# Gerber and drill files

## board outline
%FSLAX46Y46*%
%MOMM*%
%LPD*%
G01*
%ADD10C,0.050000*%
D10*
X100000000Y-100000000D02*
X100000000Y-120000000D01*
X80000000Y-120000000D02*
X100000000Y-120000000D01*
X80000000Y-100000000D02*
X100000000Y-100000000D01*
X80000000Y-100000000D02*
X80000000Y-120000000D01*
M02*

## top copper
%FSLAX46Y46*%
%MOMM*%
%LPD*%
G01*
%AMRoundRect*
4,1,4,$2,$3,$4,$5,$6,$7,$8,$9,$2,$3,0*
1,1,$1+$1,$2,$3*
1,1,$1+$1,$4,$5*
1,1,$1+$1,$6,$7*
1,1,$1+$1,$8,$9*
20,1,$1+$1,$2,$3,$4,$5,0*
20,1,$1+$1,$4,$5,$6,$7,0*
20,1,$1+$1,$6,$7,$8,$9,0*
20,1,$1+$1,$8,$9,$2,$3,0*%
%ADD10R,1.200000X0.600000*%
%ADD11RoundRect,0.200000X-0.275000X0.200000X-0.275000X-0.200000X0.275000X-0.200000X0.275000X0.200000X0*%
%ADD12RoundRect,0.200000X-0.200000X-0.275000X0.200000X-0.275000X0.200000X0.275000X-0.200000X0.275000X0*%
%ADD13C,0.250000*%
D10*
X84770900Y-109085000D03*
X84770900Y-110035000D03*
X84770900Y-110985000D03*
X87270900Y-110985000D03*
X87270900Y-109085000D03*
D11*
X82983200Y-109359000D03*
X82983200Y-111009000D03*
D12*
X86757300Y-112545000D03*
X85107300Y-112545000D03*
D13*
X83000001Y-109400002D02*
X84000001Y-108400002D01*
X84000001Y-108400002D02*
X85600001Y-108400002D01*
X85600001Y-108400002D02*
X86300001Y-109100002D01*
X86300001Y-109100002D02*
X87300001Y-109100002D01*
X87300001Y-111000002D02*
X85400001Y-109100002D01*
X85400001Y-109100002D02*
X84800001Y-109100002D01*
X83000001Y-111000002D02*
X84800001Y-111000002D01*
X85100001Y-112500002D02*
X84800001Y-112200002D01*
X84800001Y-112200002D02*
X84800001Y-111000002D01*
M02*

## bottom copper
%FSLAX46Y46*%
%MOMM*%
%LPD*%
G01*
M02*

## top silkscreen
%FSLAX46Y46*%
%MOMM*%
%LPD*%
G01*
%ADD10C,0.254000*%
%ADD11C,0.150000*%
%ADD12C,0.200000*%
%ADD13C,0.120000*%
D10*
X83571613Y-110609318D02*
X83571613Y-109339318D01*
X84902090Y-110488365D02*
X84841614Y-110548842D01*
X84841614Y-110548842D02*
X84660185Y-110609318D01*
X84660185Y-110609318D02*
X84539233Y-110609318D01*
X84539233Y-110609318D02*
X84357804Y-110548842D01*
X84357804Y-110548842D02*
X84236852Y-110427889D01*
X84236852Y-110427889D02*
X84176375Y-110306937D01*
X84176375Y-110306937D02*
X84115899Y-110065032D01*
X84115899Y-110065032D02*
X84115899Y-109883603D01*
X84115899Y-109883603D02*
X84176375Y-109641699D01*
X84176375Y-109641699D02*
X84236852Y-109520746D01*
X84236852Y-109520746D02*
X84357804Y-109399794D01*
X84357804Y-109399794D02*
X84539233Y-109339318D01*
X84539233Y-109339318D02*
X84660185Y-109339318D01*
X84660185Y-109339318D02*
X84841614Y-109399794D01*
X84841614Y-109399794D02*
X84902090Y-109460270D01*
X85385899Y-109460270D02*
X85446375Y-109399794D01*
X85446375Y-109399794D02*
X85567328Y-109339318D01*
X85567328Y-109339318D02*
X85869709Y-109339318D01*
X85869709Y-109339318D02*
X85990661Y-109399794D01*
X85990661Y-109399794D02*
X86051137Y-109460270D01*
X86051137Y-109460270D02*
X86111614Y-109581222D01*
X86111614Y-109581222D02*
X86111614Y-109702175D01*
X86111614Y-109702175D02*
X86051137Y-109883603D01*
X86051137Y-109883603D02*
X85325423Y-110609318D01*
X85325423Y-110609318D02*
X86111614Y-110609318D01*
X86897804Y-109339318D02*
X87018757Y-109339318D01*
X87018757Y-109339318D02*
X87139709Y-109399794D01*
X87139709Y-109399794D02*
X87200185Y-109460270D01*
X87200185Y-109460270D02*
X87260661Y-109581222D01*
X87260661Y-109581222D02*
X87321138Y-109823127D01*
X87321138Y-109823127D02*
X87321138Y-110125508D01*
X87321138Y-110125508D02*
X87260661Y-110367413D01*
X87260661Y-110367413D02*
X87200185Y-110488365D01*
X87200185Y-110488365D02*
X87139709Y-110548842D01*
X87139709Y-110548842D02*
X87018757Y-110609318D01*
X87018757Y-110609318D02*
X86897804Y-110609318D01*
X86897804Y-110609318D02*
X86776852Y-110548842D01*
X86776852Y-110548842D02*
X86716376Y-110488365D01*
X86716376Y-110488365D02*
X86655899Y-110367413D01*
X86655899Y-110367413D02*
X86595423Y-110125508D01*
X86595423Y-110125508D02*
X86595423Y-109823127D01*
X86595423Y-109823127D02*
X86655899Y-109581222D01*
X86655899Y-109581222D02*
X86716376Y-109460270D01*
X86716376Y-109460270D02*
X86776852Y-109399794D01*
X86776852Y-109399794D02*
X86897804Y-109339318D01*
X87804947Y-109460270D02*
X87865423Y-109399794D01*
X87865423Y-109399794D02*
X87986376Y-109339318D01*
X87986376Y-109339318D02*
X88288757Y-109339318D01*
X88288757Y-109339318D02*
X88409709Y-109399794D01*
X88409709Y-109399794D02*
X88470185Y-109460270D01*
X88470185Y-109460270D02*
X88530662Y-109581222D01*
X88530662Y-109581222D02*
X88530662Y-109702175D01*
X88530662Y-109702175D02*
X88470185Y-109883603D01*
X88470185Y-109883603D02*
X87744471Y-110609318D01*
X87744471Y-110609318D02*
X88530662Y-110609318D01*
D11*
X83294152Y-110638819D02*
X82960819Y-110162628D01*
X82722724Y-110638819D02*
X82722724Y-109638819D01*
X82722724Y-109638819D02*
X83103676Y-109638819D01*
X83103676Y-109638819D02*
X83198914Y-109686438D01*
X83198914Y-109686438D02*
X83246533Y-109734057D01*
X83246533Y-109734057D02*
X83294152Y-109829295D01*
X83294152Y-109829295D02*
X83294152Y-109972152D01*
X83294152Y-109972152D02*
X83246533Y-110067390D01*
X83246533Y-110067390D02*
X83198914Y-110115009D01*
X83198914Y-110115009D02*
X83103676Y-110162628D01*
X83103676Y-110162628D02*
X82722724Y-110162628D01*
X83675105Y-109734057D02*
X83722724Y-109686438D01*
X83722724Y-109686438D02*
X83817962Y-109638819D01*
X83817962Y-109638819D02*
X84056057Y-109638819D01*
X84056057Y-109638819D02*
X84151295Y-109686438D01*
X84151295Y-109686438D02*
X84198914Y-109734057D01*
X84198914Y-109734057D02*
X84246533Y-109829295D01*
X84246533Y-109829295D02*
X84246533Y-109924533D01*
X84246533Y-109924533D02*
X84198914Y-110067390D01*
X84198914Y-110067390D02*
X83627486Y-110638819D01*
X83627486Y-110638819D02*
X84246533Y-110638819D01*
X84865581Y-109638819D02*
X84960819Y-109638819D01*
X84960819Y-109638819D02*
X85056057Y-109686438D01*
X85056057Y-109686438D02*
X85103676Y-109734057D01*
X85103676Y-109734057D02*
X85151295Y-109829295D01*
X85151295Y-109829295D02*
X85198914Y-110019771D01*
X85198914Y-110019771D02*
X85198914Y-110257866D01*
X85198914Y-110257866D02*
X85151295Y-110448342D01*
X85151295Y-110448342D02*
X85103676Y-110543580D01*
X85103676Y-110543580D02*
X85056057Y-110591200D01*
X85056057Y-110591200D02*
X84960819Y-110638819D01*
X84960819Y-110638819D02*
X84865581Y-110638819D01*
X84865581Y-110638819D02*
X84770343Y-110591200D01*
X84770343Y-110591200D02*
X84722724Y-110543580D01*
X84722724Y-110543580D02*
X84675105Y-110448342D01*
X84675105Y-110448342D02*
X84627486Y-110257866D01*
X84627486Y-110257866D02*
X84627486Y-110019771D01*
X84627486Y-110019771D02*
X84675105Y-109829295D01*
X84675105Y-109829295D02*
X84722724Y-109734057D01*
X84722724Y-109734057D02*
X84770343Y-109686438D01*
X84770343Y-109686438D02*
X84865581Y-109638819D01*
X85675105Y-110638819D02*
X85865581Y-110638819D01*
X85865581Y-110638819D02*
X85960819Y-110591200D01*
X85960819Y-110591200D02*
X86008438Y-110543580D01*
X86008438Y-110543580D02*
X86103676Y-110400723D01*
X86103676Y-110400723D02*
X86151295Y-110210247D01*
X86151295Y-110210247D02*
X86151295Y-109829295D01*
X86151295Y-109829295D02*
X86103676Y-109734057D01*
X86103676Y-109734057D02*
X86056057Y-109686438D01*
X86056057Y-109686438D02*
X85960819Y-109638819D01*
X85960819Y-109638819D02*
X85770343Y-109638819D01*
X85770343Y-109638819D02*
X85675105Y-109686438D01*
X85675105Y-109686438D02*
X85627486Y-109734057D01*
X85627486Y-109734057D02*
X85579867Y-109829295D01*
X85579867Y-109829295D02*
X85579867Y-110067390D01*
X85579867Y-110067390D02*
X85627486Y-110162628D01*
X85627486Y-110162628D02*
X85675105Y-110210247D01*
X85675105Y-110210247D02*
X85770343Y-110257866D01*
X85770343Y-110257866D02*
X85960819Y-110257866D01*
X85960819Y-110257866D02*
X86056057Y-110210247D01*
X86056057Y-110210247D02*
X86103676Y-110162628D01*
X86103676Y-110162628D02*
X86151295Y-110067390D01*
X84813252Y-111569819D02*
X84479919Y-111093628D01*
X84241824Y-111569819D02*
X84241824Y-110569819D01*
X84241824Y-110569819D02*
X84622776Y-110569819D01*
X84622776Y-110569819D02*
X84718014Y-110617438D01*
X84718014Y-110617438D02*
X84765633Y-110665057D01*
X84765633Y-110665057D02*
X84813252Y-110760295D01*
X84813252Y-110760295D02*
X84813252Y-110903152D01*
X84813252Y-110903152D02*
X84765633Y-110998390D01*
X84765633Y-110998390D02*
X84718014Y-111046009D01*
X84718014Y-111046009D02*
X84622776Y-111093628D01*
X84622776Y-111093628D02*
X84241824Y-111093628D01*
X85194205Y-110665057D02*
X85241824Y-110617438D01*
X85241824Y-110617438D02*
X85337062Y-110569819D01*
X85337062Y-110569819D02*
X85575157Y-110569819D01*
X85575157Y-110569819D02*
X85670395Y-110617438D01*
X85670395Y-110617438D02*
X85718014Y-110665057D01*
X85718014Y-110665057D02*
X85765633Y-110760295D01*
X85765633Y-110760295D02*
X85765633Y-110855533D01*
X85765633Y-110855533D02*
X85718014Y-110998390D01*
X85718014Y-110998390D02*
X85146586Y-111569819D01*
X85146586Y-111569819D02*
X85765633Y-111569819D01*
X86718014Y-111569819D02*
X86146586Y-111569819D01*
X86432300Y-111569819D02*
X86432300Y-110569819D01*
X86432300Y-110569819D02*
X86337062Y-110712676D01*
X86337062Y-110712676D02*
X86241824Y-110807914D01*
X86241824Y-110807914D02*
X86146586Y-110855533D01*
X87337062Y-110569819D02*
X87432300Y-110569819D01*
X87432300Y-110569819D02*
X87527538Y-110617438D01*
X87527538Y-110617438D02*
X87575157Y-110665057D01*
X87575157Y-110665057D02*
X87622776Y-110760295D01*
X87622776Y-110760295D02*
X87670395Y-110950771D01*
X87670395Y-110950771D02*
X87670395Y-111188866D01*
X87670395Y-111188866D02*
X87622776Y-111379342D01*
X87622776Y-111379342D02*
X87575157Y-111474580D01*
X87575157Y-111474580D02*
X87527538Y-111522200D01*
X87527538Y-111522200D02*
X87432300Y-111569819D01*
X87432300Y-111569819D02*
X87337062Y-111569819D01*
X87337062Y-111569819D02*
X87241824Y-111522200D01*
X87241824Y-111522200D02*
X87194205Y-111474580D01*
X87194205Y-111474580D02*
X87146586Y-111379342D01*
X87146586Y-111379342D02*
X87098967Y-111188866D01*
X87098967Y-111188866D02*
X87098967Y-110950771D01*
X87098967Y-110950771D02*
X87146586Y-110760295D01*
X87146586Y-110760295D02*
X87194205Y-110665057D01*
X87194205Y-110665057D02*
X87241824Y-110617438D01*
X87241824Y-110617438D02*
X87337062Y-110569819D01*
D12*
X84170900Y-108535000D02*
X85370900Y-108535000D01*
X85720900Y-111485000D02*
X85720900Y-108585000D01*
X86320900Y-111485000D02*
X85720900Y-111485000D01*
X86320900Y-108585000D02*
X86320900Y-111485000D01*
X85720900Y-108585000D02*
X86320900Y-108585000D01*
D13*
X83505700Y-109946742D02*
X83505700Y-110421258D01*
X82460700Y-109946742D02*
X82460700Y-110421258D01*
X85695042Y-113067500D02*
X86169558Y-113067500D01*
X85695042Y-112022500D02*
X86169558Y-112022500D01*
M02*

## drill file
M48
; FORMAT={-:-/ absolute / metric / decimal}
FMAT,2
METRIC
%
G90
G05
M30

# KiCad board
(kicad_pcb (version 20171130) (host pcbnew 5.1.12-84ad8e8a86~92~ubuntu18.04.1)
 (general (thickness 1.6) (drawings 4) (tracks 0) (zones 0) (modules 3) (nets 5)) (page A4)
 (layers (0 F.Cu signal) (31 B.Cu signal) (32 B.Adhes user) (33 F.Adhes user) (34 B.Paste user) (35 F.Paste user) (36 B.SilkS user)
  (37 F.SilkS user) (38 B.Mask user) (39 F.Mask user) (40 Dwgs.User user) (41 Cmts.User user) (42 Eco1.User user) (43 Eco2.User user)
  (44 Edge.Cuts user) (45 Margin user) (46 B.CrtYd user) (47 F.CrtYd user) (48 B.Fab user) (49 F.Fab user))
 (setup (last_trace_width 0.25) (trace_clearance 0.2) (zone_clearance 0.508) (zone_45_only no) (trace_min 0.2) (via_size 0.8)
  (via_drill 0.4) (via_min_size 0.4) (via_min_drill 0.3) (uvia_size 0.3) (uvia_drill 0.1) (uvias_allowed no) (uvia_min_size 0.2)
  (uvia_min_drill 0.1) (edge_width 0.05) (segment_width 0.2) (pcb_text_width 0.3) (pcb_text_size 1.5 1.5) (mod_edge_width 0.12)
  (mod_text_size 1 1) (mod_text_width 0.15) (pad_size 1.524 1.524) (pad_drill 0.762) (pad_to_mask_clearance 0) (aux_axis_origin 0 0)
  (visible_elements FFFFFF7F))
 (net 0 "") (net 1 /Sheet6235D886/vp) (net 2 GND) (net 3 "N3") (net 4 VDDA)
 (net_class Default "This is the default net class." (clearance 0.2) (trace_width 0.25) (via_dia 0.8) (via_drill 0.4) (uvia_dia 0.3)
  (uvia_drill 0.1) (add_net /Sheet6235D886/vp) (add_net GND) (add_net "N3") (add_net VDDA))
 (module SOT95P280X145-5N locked (layer F.Cu) (at 86.020900 110.035000)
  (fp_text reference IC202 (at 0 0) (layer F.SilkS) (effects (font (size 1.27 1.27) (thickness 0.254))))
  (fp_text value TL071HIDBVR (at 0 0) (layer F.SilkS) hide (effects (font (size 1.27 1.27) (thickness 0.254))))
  (fp_line (start -1.85 -1.5) (end -0.65 -1.5) (layer F.SilkS) (width 0.2))
  (fp_line (start -0.3 1.45) (end -0.3 -1.45) (layer F.SilkS) (width 0.2))
  (fp_line (start 0.3 1.45) (end -0.3 1.45) (layer F.SilkS) (width 0.2))
  (fp_line (start 0.3 -1.45) (end 0.3 1.45) (layer F.SilkS) (width 0.2))
  (fp_line (start -0.3 -1.45) (end 0.3 -1.45) (layer F.SilkS) (width 0.2))
  (pad 1 smd rect (at -1.25 -0.95 90.000000) (size 0.6 1.2) (layers F.Cu F.Mask F.Paste) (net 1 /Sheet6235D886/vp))
  (pad 2 smd rect (at -1.25 0 90.000000) (size 0.6 1.2) (layers F.Cu F.Mask F.Paste) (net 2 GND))
  (pad 3 smd rect (at -1.25 0.95 90.000000) (size 0.6 1.2) (layers F.Cu F.Mask F.Paste) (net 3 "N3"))
  (pad 4 smd rect (at 1.25 0.95 90.000000) (size 0.6 1.2) (layers F.Cu F.Mask F.Paste) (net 1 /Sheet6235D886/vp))
  (pad 5 smd rect (at 1.25 -0.95 90.000000) (size 0.6 1.2) (layers F.Cu F.Mask F.Paste) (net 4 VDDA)))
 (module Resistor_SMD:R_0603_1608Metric (layer F.Cu) (at 82.983200 110.184000 270.000000)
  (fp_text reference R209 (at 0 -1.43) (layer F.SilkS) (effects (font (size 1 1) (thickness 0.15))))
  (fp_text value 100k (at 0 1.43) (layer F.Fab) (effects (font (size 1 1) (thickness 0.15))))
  (fp_line (start -0.237258 -0.5225) (end 0.237258 -0.5225) (layer F.SilkS) (width 0.12))
  (fp_line (start -0.237258 0.5225) (end 0.237258 0.5225) (layer F.SilkS) (width 0.12))
  (pad 1 smd roundrect (at -0.825 0 270.000000) (size 0.8 0.95) (layers F.Cu F.Mask F.Paste) (roundrect_rratio 0.25) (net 4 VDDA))
  (pad 2 smd roundrect (at 0.825 0 270.000000) (size 0.8 0.95) (layers F.Cu F.Mask F.Paste) (roundrect_rratio 0.25) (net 3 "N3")))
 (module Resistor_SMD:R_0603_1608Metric (layer F.Cu) (at 85.932300 112.545000)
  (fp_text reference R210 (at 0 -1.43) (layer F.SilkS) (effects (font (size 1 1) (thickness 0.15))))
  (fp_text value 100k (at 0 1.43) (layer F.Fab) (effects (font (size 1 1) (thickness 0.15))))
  (fp_line (start -0.237258 0.5225) (end 0.237258 0.5225) (layer F.SilkS) (width 0.12))
  (fp_line (start -0.237258 -0.5225) (end 0.237258 -0.5225) (layer F.SilkS) (width 0.12))
  (pad 2 smd roundrect (at 0.825 0) (size 0.8 0.95) (layers F.Cu F.Mask F.Paste) (roundrect_rratio 0.25) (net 2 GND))
  (pad 1 smd roundrect (at -0.825 0) (size 0.8 0.95) (layers F.Cu F.Mask F.Paste) (roundrect_rratio 0.25) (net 3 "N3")))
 (gr_line (start 100 100) (end 100 120) (layer Edge.Cuts) (width 0.05))
 (gr_line (start 80 120) (end 100 120) (layer Edge.Cuts) (width 0.05))
 (gr_line (start 80 100) (end 100 100) (layer Edge.Cuts) (width 0.05))
 (gr_line (start 80 100) (end 80 120) (layer Edge.Cuts) (width 0.05))
 (segment (start 83.000001 109.400002) (end 84.000001 108.400002) (width 0.250000) (layer F.Cu) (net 4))
 (segment (start 84.000001 108.400002) (end 85.600001 108.400002) (width 0.250000) (layer F.Cu) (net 4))
 (segment (start 85.600001 108.400002) (end 86.300001 109.100002) (width 0.250000) (layer F.Cu) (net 4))
 (segment (start 86.300001 109.100002) (end 87.300001 109.100002) (width 0.250000) (layer F.Cu) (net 4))
 (segment (start 87.300001 111.000002) (end 85.400001 109.100002) (width 0.250000) (layer F.Cu) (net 1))
 (segment (start 85.400001 109.100002) (end 84.800001 109.100002) (width 0.250000) (layer F.Cu) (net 1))
 (segment (start 83.000001 111.000002) (end 84.800001 111.000002) (width 0.250000) (layer F.Cu) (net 3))
 (segment (start 85.100001 112.500002) (end 84.800001 112.200002) (width 0.250000) (layer F.Cu) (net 3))
 (segment (start 84.800001 112.200002) (end 84.800001 111.000002) (width 0.250000) (layer F.Cu) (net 3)))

